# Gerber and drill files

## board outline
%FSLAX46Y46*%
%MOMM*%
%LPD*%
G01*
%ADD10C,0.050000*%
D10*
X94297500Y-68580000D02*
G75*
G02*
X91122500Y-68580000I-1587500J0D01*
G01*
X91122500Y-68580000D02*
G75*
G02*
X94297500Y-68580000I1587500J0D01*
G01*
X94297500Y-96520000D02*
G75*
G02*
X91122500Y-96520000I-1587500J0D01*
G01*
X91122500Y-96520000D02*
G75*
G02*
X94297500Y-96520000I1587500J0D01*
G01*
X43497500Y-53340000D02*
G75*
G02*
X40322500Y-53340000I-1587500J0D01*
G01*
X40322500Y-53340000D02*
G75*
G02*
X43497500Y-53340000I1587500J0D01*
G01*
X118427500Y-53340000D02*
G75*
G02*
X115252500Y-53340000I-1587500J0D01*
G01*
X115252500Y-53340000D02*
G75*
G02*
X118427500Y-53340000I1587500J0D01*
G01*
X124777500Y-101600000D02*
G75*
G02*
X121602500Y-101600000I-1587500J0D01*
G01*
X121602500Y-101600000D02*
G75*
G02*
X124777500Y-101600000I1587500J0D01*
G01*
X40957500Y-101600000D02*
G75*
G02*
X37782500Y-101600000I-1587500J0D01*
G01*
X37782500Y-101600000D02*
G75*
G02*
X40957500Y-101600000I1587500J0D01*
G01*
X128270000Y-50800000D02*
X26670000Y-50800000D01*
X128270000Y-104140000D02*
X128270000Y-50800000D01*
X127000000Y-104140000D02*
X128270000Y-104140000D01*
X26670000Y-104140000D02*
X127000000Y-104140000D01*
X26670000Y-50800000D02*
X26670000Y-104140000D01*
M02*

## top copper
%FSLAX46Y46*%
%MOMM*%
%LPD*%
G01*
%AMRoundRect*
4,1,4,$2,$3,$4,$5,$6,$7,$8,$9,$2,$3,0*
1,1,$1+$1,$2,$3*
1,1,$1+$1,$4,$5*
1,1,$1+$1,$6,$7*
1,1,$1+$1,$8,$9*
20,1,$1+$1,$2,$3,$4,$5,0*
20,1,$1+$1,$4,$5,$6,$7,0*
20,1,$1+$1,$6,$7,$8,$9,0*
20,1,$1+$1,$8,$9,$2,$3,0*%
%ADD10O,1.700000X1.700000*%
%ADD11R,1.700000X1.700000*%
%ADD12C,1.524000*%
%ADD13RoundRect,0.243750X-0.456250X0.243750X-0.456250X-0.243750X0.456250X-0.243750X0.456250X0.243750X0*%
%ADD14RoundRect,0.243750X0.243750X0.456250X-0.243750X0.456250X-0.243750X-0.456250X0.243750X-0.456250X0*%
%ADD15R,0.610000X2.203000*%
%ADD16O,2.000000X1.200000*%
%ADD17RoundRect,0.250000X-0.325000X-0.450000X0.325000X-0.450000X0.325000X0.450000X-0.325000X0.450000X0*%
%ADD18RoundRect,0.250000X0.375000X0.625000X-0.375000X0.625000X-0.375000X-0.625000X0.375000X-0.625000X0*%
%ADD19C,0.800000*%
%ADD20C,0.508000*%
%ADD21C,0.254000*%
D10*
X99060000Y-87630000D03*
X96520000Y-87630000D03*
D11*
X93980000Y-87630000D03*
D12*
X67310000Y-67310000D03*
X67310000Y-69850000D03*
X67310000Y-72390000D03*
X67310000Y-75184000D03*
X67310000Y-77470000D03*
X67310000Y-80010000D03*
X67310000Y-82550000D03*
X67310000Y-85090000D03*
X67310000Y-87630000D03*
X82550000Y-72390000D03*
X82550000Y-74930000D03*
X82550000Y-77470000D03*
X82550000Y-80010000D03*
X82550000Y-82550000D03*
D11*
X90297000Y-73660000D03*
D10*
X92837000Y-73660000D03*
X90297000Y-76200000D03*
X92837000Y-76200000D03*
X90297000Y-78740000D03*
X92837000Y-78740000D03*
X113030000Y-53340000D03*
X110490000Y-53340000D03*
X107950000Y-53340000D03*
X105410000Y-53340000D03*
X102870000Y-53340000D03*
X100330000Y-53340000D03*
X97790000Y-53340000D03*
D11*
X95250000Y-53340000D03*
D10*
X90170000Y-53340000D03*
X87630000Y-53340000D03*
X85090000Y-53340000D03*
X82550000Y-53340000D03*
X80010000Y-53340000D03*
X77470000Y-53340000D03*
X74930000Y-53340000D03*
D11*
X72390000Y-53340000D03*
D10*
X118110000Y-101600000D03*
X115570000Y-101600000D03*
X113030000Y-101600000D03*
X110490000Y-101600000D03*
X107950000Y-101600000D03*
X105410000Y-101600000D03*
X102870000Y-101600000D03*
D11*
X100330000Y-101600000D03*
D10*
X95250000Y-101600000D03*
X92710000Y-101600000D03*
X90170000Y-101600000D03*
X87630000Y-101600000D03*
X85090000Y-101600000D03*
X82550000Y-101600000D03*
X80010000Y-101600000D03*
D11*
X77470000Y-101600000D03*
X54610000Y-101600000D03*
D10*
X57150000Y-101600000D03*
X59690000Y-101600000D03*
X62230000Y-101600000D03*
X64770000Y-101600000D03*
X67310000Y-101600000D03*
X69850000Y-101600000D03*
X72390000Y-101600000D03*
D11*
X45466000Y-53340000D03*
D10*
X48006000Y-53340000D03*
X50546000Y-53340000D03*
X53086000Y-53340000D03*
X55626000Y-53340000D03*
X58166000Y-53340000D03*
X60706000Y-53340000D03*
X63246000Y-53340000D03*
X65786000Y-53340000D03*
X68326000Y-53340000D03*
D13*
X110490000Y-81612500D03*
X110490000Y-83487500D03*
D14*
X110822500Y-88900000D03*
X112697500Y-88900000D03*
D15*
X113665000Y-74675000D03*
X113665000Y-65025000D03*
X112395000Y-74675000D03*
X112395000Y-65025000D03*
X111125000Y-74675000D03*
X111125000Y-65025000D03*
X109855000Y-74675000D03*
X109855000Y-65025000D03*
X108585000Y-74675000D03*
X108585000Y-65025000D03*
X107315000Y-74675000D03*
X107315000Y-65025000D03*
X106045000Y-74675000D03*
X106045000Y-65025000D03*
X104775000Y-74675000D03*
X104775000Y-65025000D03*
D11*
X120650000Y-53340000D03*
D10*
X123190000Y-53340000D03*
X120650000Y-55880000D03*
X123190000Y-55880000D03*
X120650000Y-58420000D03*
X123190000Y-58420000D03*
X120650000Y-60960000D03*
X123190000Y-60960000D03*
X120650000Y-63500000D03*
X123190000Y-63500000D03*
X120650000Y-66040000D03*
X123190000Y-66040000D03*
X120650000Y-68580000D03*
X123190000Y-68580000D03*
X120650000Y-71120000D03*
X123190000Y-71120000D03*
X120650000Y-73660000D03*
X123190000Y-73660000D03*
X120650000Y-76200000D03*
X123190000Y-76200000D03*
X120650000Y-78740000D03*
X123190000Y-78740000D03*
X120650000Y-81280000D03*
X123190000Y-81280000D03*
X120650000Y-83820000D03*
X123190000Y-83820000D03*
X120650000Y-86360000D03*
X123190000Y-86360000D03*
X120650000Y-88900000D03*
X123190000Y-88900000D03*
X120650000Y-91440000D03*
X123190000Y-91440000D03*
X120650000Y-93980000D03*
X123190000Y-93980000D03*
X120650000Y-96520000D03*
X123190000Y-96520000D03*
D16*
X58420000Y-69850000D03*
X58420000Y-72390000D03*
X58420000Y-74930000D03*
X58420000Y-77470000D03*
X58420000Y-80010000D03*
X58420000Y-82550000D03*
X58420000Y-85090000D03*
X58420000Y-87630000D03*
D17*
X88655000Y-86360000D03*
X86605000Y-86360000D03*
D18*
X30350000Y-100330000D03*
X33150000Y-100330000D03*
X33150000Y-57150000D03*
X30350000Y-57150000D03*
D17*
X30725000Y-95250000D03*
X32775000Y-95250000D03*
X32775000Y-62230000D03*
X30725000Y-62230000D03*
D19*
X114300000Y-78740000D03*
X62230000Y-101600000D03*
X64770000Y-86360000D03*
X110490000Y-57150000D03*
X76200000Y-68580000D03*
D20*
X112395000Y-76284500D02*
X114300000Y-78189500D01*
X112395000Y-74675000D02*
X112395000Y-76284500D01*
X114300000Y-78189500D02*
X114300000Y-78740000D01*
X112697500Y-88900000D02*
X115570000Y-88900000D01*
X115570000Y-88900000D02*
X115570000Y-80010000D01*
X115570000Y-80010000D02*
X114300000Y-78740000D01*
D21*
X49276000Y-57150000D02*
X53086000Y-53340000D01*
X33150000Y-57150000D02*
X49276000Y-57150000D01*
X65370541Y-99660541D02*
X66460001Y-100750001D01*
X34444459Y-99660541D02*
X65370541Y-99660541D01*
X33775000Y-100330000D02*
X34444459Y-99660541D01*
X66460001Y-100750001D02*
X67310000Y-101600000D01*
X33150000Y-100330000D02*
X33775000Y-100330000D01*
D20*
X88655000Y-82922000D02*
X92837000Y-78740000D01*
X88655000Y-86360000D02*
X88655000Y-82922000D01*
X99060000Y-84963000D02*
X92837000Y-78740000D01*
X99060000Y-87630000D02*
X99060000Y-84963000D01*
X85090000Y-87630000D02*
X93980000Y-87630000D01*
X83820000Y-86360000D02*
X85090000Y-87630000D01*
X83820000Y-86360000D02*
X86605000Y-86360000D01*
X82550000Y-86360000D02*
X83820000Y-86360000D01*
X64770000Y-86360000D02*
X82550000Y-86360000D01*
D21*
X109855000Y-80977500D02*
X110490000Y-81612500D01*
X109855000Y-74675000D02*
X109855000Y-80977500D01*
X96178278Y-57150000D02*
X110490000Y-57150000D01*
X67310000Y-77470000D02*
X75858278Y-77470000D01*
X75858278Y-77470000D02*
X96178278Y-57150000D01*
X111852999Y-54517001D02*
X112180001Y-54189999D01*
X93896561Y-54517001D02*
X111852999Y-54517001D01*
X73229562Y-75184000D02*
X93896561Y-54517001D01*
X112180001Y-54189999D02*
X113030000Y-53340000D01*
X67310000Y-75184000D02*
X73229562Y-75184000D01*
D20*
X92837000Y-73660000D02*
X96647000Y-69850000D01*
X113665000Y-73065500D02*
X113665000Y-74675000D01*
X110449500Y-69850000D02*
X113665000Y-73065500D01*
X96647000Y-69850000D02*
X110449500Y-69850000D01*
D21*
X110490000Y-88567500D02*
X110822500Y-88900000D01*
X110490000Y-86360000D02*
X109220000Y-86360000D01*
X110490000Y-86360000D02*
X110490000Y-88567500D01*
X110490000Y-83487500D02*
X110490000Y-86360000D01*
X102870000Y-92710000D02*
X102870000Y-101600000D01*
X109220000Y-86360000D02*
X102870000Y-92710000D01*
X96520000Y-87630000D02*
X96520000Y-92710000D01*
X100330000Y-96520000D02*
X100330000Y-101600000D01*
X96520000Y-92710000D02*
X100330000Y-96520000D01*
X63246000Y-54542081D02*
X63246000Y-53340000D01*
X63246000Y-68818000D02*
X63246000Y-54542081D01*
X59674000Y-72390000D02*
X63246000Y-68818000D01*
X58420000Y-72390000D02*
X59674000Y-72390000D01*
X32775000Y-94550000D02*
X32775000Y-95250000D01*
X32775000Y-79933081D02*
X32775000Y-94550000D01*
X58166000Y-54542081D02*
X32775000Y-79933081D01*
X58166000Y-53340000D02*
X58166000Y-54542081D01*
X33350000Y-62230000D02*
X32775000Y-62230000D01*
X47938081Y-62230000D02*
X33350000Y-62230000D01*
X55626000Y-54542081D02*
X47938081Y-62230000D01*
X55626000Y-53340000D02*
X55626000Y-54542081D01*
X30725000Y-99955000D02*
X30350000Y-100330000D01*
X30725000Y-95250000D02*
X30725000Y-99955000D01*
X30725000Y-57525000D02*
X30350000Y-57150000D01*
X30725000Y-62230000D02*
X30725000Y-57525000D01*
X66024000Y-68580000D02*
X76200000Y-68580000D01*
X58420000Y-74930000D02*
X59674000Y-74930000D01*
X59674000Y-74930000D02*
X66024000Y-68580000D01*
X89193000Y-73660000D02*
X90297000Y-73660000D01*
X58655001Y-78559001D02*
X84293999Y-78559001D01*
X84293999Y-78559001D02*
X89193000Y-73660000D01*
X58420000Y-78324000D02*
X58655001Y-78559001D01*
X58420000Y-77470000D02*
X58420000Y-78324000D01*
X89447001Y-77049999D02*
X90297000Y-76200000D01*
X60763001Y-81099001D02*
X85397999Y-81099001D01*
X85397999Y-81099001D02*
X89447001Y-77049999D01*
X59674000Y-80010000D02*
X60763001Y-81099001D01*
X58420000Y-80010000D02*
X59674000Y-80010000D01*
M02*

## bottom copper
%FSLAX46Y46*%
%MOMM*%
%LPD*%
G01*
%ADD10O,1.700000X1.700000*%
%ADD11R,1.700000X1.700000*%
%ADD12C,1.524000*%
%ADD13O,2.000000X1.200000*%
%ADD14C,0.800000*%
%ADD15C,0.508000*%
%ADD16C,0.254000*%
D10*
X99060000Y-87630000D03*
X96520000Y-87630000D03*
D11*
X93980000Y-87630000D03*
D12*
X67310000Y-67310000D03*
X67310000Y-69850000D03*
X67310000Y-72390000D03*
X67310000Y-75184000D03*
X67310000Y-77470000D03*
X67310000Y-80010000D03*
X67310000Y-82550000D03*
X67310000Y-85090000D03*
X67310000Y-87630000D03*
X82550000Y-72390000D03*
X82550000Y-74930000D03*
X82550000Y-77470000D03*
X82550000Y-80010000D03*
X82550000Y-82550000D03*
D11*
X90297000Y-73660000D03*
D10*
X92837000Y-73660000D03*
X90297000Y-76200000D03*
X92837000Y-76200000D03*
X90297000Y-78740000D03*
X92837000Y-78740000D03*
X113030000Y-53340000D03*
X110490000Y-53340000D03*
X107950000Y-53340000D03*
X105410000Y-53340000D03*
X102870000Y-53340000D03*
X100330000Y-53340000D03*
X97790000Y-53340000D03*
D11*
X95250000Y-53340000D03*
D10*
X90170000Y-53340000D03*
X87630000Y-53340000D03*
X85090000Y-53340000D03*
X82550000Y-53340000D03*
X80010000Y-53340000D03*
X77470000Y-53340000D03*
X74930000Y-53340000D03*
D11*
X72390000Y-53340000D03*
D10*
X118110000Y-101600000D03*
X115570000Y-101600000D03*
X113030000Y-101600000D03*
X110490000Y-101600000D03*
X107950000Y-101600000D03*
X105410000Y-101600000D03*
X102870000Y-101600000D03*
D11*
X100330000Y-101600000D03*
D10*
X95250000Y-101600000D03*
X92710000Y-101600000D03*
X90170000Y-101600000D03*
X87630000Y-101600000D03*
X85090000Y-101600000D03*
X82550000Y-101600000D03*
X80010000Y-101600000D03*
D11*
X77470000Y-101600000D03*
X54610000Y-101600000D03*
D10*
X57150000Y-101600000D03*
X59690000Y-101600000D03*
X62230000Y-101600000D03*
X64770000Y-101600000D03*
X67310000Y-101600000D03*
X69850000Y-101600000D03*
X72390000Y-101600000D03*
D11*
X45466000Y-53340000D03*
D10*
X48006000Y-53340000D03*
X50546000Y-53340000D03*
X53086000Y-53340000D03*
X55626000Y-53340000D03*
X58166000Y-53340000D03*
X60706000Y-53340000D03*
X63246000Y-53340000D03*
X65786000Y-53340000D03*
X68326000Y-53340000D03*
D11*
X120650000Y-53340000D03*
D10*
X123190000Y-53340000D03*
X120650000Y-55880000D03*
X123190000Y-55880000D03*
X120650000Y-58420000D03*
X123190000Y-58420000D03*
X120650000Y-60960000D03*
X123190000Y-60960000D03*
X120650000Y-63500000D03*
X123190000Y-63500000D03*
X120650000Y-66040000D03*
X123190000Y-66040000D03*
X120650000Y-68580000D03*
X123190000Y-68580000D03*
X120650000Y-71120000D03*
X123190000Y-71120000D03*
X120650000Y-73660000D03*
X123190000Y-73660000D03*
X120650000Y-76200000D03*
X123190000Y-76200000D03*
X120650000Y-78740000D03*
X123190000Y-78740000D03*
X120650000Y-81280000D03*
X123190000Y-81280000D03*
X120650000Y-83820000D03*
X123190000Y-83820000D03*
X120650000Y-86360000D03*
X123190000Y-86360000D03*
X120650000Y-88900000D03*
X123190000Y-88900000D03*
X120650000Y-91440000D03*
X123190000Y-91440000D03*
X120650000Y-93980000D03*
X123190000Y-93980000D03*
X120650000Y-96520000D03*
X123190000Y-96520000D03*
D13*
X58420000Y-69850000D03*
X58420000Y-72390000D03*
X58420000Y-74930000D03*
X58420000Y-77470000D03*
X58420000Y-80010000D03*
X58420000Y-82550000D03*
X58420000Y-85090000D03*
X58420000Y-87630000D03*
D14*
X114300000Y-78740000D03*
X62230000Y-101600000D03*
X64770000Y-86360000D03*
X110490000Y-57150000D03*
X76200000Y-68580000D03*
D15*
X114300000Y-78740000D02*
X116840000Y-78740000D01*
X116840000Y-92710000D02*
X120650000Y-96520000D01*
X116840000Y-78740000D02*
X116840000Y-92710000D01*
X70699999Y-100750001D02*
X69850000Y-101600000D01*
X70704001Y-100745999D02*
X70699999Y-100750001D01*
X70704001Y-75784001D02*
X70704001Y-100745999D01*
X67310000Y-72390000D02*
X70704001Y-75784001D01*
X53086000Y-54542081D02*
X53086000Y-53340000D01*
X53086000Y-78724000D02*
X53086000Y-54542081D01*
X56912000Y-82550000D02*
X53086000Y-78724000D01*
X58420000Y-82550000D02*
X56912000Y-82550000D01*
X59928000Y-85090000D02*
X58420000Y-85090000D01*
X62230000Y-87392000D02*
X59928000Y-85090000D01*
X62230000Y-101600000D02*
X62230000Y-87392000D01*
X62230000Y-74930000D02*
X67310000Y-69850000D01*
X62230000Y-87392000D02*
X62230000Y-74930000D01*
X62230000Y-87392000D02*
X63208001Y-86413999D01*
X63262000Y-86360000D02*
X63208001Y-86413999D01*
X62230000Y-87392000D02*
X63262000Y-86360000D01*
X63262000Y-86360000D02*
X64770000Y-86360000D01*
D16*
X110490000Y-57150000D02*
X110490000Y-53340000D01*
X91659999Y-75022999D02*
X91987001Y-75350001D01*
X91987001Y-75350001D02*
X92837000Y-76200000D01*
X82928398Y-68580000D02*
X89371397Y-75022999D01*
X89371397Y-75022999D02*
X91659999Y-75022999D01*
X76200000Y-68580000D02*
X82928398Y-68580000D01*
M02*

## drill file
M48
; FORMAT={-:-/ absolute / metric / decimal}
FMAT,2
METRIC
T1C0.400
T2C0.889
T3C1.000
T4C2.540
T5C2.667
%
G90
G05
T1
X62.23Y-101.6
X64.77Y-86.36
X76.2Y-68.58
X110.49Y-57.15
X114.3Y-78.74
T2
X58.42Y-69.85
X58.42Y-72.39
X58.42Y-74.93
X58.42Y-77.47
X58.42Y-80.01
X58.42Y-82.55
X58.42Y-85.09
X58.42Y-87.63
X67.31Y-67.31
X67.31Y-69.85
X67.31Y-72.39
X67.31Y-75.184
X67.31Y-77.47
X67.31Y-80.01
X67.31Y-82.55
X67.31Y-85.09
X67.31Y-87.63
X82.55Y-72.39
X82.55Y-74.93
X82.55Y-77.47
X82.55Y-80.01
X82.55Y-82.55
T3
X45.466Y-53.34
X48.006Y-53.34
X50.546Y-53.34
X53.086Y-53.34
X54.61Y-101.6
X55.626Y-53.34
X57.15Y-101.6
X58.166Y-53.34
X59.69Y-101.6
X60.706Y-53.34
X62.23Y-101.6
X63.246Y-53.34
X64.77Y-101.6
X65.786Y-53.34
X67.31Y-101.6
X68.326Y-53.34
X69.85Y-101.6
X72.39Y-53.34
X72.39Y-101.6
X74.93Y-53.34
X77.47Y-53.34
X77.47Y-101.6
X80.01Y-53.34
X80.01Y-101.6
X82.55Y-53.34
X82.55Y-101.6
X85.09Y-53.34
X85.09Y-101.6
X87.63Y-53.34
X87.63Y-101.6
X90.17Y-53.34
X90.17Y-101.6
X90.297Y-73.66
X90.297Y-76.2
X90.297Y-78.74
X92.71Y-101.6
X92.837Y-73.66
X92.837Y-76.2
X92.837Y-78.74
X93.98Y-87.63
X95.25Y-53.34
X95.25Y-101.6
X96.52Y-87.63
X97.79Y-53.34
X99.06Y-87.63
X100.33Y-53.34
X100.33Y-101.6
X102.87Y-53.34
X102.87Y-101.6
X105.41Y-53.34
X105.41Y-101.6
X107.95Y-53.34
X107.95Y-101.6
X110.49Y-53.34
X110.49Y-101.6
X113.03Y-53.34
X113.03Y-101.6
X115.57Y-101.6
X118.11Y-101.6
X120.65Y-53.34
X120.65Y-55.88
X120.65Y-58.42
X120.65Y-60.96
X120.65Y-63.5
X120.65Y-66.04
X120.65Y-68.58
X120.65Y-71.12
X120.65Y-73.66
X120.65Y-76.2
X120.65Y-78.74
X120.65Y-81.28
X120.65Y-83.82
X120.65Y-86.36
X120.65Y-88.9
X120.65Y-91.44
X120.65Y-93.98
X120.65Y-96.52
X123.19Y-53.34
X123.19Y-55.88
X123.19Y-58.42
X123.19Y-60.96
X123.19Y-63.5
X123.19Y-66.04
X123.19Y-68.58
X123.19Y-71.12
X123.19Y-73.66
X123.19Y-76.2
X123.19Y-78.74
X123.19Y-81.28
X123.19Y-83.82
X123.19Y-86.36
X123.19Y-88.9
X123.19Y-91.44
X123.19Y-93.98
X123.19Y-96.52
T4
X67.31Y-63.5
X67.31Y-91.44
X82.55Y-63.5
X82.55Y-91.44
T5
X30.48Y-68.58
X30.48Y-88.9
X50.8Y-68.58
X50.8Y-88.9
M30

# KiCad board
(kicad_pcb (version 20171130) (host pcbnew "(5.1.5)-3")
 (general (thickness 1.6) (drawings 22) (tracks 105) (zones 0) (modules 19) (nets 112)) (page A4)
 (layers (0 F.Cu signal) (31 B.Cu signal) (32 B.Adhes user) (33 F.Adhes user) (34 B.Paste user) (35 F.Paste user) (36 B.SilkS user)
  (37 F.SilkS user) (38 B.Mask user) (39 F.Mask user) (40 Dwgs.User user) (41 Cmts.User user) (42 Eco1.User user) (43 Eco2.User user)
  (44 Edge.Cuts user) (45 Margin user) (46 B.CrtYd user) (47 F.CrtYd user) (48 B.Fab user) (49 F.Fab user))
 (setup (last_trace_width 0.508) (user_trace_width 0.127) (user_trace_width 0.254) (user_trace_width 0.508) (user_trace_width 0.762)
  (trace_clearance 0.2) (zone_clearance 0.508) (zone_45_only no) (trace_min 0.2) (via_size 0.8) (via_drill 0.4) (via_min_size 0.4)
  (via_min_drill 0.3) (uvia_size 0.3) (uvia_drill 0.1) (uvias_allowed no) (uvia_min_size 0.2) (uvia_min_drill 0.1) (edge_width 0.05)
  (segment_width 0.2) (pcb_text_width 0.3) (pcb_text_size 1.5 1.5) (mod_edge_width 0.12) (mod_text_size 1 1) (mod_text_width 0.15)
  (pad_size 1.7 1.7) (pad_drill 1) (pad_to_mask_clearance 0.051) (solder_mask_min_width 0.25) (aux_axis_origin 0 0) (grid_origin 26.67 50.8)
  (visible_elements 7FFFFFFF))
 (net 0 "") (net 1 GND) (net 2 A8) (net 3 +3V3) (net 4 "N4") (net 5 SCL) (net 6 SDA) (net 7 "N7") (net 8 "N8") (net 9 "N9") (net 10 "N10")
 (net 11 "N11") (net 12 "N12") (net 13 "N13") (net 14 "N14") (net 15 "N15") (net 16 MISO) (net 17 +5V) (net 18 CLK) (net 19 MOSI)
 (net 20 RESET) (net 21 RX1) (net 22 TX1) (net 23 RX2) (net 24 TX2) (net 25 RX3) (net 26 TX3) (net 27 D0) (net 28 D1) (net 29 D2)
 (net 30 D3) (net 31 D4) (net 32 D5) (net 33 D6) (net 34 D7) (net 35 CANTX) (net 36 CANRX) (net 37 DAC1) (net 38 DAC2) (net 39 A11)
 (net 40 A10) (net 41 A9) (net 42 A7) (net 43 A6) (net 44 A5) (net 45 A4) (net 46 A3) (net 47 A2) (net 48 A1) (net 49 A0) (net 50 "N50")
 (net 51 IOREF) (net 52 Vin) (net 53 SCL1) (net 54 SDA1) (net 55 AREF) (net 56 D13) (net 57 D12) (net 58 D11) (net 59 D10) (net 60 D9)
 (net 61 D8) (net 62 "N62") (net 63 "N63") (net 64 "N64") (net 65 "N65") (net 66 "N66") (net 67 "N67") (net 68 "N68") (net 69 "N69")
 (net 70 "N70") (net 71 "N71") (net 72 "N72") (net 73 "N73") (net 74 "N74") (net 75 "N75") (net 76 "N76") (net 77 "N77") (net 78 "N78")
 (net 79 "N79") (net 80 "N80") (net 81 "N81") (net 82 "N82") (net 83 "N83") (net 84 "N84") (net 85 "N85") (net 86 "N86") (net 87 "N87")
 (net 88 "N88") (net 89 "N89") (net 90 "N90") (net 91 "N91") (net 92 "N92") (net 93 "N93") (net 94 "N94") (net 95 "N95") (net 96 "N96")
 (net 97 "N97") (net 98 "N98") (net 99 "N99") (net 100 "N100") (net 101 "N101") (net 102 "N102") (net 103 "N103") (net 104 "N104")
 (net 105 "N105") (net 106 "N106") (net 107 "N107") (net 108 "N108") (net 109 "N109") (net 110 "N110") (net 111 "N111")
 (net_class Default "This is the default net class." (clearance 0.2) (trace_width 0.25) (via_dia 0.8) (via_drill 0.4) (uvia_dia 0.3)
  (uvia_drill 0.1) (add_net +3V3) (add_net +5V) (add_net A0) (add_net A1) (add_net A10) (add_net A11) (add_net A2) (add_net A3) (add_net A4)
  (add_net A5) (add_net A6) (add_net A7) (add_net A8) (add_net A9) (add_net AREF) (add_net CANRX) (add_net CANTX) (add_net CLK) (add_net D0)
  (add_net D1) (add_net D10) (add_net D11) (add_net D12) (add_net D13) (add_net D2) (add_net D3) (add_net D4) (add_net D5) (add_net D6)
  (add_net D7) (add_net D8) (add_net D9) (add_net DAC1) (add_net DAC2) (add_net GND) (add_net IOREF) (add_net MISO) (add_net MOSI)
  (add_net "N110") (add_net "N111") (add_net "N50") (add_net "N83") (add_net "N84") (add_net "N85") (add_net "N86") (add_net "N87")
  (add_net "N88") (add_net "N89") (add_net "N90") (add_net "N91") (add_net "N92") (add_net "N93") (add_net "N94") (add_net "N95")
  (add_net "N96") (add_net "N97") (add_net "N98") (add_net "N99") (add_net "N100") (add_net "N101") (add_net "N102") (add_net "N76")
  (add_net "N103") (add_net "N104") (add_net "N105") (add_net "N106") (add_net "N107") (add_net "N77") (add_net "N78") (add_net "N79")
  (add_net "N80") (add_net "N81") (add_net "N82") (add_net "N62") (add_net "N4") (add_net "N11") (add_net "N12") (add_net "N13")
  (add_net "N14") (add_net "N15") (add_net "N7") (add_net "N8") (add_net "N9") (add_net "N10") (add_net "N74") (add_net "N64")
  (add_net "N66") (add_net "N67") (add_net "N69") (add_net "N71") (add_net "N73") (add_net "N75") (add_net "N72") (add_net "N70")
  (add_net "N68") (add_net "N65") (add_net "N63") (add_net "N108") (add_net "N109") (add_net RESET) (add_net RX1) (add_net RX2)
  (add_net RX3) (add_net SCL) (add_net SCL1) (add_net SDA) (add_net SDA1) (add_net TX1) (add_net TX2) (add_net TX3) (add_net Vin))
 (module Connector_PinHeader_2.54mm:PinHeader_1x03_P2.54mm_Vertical (layer F.Cu) (at 93.98 87.63 90)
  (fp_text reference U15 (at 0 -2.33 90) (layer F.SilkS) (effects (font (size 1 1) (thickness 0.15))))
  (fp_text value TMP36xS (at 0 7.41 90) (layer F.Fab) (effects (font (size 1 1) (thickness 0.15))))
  (pad 3 thru_hole oval (at 0 5.08 90) (size 1.7 1.7) (drill 1) (layers *.Cu *.Mask) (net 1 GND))
  (pad 2 thru_hole oval (at 0 2.54 90) (size 1.7 1.7) (drill 1) (layers *.Cu *.Mask) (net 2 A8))
  (pad 1 thru_hole rect (at 0 0 90) (size 1.7 1.7) (drill 1) (layers *.Cu *.Mask) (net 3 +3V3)))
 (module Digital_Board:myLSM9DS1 (layer F.Cu) (at 74.93 77.47)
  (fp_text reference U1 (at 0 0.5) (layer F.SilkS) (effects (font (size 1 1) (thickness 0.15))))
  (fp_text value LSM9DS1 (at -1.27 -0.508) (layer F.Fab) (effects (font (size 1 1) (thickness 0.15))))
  (pad 1 thru_hole circle (at -7.62 -10.16) (size 1.524 1.524) (drill 0.889) (layers *.Cu *.Mask) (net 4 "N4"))
  (pad 2 thru_hole circle (at -7.62 -7.62) (size 1.524 1.524) (drill 0.889) (layers *.Cu *.Mask) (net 3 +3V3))
  (pad 3 thru_hole circle (at -7.62 -5.08) (size 1.524 1.524) (drill 0.889) (layers *.Cu *.Mask) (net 1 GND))
  (pad 4 thru_hole circle (at -7.62 -2.286) (size 1.524 1.524) (drill 0.889) (layers *.Cu *.Mask) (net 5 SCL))
  (pad 5 thru_hole circle (at -7.62 0) (size 1.524 1.524) (drill 0.889) (layers *.Cu *.Mask) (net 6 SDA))
  (pad 6 thru_hole circle (at -7.62 2.54) (size 1.524 1.524) (drill 0.889) (layers *.Cu *.Mask) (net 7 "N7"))
  (pad 7 thru_hole circle (at -7.62 5.08) (size 1.524 1.524) (drill 0.889) (layers *.Cu *.Mask) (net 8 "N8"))
  (pad 8 thru_hole circle (at -7.62 7.62) (size 1.524 1.524) (drill 0.889) (layers *.Cu *.Mask) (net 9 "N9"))
  (pad 9 thru_hole circle (at -7.62 10.16) (size 1.524 1.524) (drill 0.889) (layers *.Cu *.Mask Eco2.User) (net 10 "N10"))
  (pad 10 thru_hole circle (at 7.62 -5.08) (size 1.524 1.524) (drill 0.889) (layers *.Cu *.Mask) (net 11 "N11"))
  (pad 11 thru_hole circle (at 7.62 -2.54) (size 1.524 1.524) (drill 0.889) (layers *.Cu *.Mask) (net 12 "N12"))
  (pad 12 thru_hole circle (at 7.62 0) (size 1.524 1.524) (drill 0.889) (layers *.Cu *.Mask) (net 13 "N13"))
  (pad 13 thru_hole circle (at 7.62 2.54) (size 1.524 1.524) (drill 0.889) (layers *.Cu *.Mask) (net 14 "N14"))
  (pad 14 thru_hole circle (at 7.62 5.08) (size 1.524 1.524) (drill 0.889) (layers *.Cu *.Mask) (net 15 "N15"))
  (pad "" np_thru_hole circle (at -7.62 -13.97) (size 2.54 2.54) (drill 2.54) (layers *.Cu *.Mask))
  (pad "" np_thru_hole circle (at 7.62 -13.97) (size 2.54 2.54) (drill 2.54) (layers *.Cu *.Mask))
  (pad "" np_thru_hole circle (at -7.62 13.97) (size 2.54 2.54) (drill 2.54) (layers *.Cu *.Mask))
  (pad "" np_thru_hole circle (at 7.62 13.97) (size 2.54 2.54) (drill 2.54) (layers *.Cu *.Mask)))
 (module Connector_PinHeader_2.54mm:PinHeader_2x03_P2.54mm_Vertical (layer F.Cu) (at 90.297 73.66)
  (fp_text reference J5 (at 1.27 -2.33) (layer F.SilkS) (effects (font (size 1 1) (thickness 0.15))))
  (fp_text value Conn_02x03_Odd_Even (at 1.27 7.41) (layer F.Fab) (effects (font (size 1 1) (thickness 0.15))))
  (pad 1 thru_hole rect (at 0 0) (size 1.7 1.7) (drill 1) (layers *.Cu *.Mask) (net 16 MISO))
  (pad 2 thru_hole oval (at 2.54 0) (size 1.7 1.7) (drill 1) (layers *.Cu *.Mask) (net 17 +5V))
  (pad 3 thru_hole oval (at 0 2.54) (size 1.7 1.7) (drill 1) (layers *.Cu *.Mask) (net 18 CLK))
  (pad 4 thru_hole oval (at 2.54 2.54) (size 1.7 1.7) (drill 1) (layers *.Cu *.Mask) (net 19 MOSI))
  (pad 5 thru_hole oval (at 0 5.08) (size 1.7 1.7) (drill 1) (layers *.Cu *.Mask) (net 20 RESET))
  (pad 6 thru_hole oval (at 2.54 5.08) (size 1.7 1.7) (drill 1) (layers *.Cu *.Mask) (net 1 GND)))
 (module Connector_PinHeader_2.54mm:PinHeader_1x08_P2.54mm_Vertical (layer F.Cu) (at 95.25 53.34 90)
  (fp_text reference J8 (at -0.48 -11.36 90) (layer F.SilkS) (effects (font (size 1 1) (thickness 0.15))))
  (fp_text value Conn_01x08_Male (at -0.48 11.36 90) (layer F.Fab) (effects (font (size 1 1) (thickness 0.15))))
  (pad 8 thru_hole oval (at 0 17.78 90) (size 1.7 1.7) (drill 1) (layers *.Cu *.Mask) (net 5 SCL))
  (pad 7 thru_hole oval (at 0 15.24 90) (size 1.7 1.7) (drill 1) (layers *.Cu *.Mask) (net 6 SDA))
  (pad 6 thru_hole oval (at 0 12.7 90) (size 1.7 1.7) (drill 1) (layers *.Cu *.Mask) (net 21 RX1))
  (pad 5 thru_hole oval (at 0 10.16 90) (size 1.7 1.7) (drill 1) (layers *.Cu *.Mask) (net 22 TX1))
  (pad 4 thru_hole oval (at 0 7.62 90) (size 1.7 1.7) (drill 1) (layers *.Cu *.Mask) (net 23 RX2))
  (pad 3 thru_hole oval (at 0 5.08 90) (size 1.7 1.7) (drill 1) (layers *.Cu *.Mask) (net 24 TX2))
  (pad 2 thru_hole oval (at 0 2.54 90) (size 1.7 1.7) (drill 1) (layers *.Cu *.Mask) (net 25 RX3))
  (pad 1 thru_hole rect (at 0 0 90) (size 1.7 1.7) (drill 1) (layers *.Cu *.Mask) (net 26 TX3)))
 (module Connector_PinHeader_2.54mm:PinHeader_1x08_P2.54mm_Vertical (layer F.Cu) (at 72.39 53.34 90)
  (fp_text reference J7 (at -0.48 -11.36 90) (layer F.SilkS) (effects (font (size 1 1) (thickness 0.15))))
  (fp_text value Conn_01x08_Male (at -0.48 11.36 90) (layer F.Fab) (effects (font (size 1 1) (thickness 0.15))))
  (pad 8 thru_hole oval (at 0 17.78 90) (size 1.7 1.7) (drill 1) (layers *.Cu *.Mask) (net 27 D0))
  (pad 7 thru_hole oval (at 0 15.24 90) (size 1.7 1.7) (drill 1) (layers *.Cu *.Mask) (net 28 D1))
  (pad 6 thru_hole oval (at 0 12.7 90) (size 1.7 1.7) (drill 1) (layers *.Cu *.Mask) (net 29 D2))
  (pad 5 thru_hole oval (at 0 10.16 90) (size 1.7 1.7) (drill 1) (layers *.Cu *.Mask) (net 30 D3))
  (pad 4 thru_hole oval (at 0 7.62 90) (size 1.7 1.7) (drill 1) (layers *.Cu *.Mask) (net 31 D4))
  (pad 3 thru_hole oval (at 0 5.08 90) (size 1.7 1.7) (drill 1) (layers *.Cu *.Mask) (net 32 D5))
  (pad 2 thru_hole oval (at 0 2.54 90) (size 1.7 1.7) (drill 1) (layers *.Cu *.Mask) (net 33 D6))
  (pad 1 thru_hole rect (at 0 0 90) (size 1.7 1.7) (drill 1) (layers *.Cu *.Mask) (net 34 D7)))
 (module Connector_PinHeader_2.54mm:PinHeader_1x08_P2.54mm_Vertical (layer F.Cu) (at 100.33 101.6 90)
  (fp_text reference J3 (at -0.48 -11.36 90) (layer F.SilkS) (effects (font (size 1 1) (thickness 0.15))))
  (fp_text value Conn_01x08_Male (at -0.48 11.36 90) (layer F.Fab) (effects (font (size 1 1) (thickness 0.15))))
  (pad 8 thru_hole oval (at 0 17.78 90) (size 1.7 1.7) (drill 1) (layers *.Cu *.Mask) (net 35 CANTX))
  (pad 7 thru_hole oval (at 0 15.24 90) (size 1.7 1.7) (drill 1) (layers *.Cu *.Mask) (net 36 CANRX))
  (pad 6 thru_hole oval (at 0 12.7 90) (size 1.7 1.7) (drill 1) (layers *.Cu *.Mask) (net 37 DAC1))
  (pad 5 thru_hole oval (at 0 10.16 90) (size 1.7 1.7) (drill 1) (layers *.Cu *.Mask) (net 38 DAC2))
  (pad 4 thru_hole oval (at 0 7.62 90) (size 1.7 1.7) (drill 1) (layers *.Cu *.Mask) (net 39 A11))
  (pad 3 thru_hole oval (at 0 5.08 90) (size 1.7 1.7) (drill 1) (layers *.Cu *.Mask) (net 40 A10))
  (pad 2 thru_hole oval (at 0 2.54 90) (size 1.7 1.7) (drill 1) (layers *.Cu *.Mask) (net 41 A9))
  (pad 1 thru_hole rect (at 0 0 90) (size 1.7 1.7) (drill 1) (layers *.Cu *.Mask) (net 2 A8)))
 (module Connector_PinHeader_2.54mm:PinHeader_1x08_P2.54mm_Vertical (layer F.Cu) (at 77.47 101.6 90)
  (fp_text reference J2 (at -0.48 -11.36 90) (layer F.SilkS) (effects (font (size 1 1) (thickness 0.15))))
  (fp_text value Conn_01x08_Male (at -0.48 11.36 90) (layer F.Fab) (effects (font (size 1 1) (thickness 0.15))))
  (pad 8 thru_hole oval (at 0 17.78 90) (size 1.7 1.7) (drill 1) (layers *.Cu *.Mask) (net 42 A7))
  (pad 7 thru_hole oval (at 0 15.24 90) (size 1.7 1.7) (drill 1) (layers *.Cu *.Mask) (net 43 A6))
  (pad 6 thru_hole oval (at 0 12.7 90) (size 1.7 1.7) (drill 1) (layers *.Cu *.Mask) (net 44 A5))
  (pad 5 thru_hole oval (at 0 10.16 90) (size 1.7 1.7) (drill 1) (layers *.Cu *.Mask) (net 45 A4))
  (pad 4 thru_hole oval (at 0 7.62 90) (size 1.7 1.7) (drill 1) (layers *.Cu *.Mask) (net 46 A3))
  (pad 3 thru_hole oval (at 0 5.08 90) (size 1.7 1.7) (drill 1) (layers *.Cu *.Mask) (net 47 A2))
  (pad 2 thru_hole oval (at 0 2.54 90) (size 1.7 1.7) (drill 1) (layers *.Cu *.Mask) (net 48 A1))
  (pad 1 thru_hole rect (at 0 0 90) (size 1.7 1.7) (drill 1) (layers *.Cu *.Mask) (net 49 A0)))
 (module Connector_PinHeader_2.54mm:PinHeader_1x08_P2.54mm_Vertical (layer F.Cu) (at 54.61 101.6 90)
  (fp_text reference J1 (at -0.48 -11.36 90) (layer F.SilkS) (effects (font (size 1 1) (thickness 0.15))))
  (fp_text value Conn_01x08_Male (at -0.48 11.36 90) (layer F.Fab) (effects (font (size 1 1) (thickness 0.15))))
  (pad 1 thru_hole rect (at 0 0 90) (size 1.7 1.7) (drill 1) (layers *.Cu *.Mask) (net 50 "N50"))
  (pad 2 thru_hole oval (at 0 2.54 90) (size 1.7 1.7) (drill 1) (layers *.Cu *.Mask) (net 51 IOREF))
  (pad 3 thru_hole oval (at 0 5.08 90) (size 1.7 1.7) (drill 1) (layers *.Cu *.Mask) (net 20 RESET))
  (pad 4 thru_hole oval (at 0 7.62 90) (size 1.7 1.7) (drill 1) (layers *.Cu *.Mask) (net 3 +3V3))
  (pad 5 thru_hole oval (at 0 10.16 90) (size 1.7 1.7) (drill 1) (layers *.Cu *.Mask) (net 17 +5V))
  (pad 6 thru_hole oval (at 0 12.7 90) (size 1.7 1.7) (drill 1) (layers *.Cu *.Mask) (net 1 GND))
  (pad 7 thru_hole oval (at 0 15.24 90) (size 1.7 1.7) (drill 1) (layers *.Cu *.Mask) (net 1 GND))
  (pad 8 thru_hole oval (at 0 17.78 90) (size 1.7 1.7) (drill 1) (layers *.Cu *.Mask) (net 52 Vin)))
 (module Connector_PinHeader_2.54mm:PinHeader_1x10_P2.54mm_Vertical (layer F.Cu) (at 45.466 53.34 90)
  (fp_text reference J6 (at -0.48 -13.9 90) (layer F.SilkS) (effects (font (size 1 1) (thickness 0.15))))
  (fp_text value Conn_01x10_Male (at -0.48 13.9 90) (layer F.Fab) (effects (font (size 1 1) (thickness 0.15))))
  (pad 1 thru_hole rect (at 0 0 90) (size 1.7 1.7) (drill 1) (layers *.Cu *.Mask) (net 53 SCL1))
  (pad 2 thru_hole oval (at 0 2.54 90) (size 1.7 1.7) (drill 1) (layers *.Cu *.Mask) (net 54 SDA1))
  (pad 3 thru_hole oval (at 0 5.08 90) (size 1.7 1.7) (drill 1) (layers *.Cu *.Mask) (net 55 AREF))
  (pad 4 thru_hole oval (at 0 7.62 90) (size 1.7 1.7) (drill 1) (layers *.Cu *.Mask) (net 1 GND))
  (pad 5 thru_hole oval (at 0 10.16 90) (size 1.7 1.7) (drill 1) (layers *.Cu *.Mask) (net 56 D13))
  (pad 6 thru_hole oval (at 0 12.7 90) (size 1.7 1.7) (drill 1) (layers *.Cu *.Mask) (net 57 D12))
  (pad 7 thru_hole oval (at 0 15.24 90) (size 1.7 1.7) (drill 1) (layers *.Cu *.Mask) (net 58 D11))
  (pad 8 thru_hole oval (at 0 17.78 90) (size 1.7 1.7) (drill 1) (layers *.Cu *.Mask) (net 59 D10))
  (pad 9 thru_hole oval (at 0 20.32 90) (size 1.7 1.7) (drill 1) (layers *.Cu *.Mask) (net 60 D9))
  (pad 10 thru_hole oval (at 0 22.86 90) (size 1.7 1.7) (drill 1) (layers *.Cu *.Mask) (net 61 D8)))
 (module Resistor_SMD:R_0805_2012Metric (layer F.Cu) (at 110.49 82.55 270)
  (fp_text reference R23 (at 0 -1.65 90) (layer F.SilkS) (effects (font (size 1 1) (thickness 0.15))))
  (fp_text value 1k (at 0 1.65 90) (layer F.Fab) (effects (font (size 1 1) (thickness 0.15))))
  (pad 1 smd roundrect (at -0.9375 0 270) (size 0.975 1.4) (layers F.Cu F.Paste F.Mask) (roundrect_rratio 0.25) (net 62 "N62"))
  (pad 2 smd roundrect (at 0.9375 0 270) (size 0.975 1.4) (layers F.Cu F.Paste F.Mask) (roundrect_rratio 0.25) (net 41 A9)))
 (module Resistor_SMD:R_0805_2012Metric (layer F.Cu) (at 111.76 88.9 180)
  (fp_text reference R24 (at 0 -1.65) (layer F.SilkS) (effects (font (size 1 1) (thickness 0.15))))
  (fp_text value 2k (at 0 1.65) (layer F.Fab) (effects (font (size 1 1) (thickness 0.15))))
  (pad 2 smd roundrect (at 0.9375 0 180) (size 0.975 1.4) (layers F.Cu F.Paste F.Mask) (roundrect_rratio 0.25) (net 41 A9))
  (pad 1 smd roundrect (at -0.9375 0 180) (size 0.975 1.4) (layers F.Cu F.Paste F.Mask) (roundrect_rratio 0.25) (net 1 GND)))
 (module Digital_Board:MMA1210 (layer F.Cu) (at 109.22 69.85)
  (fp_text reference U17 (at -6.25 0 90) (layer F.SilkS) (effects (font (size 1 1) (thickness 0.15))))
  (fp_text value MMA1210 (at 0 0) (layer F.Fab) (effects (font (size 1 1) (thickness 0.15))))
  (pad 8 smd rect (at 4.445 4.825) (size 0.61 2.203) (layers F.Cu F.Paste F.Mask) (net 17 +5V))
  (pad 9 smd rect (at 4.445 -4.825) (size 0.61 2.203) (layers F.Cu F.Paste F.Mask) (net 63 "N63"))
  (pad 7 smd rect (at 3.175 4.825) (size 0.61 2.203) (layers F.Cu F.Paste F.Mask) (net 1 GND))
  (pad 10 smd rect (at 3.175 -4.825) (size 0.61 2.203) (layers F.Cu F.Paste F.Mask) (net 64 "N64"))
  (pad 6 smd rect (at 1.905 4.825) (size 0.61 2.203) (layers F.Cu F.Paste F.Mask) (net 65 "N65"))
  (pad 11 smd rect (at 1.905 -4.825) (size 0.61 2.203) (layers F.Cu F.Paste F.Mask) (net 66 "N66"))
  (pad 5 smd rect (at 0.635 4.825) (size 0.61 2.203) (layers F.Cu F.Paste F.Mask) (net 62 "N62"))
  (pad 12 smd rect (at 0.635 -4.825) (size 0.61 2.203) (layers F.Cu F.Paste F.Mask) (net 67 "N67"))
  (pad 4 smd rect (at -0.635 4.825) (size 0.61 2.203) (layers F.Cu F.Paste F.Mask) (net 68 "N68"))
  (pad 13 smd rect (at -0.635 -4.825) (size 0.61 2.203) (layers F.Cu F.Paste F.Mask) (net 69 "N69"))
  (pad 3 smd rect (at -1.905 4.825) (size 0.61 2.203) (layers F.Cu F.Paste F.Mask) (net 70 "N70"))
  (pad 14 smd rect (at -1.905 -4.825) (size 0.61 2.203) (layers F.Cu F.Paste F.Mask) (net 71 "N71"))
  (pad 2 smd rect (at -3.175 4.825) (size 0.61 2.203) (layers F.Cu F.Paste F.Mask) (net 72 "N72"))
  (pad 15 smd rect (at -3.175 -4.825) (size 0.61 2.203) (layers F.Cu F.Paste F.Mask) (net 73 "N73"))
  (pad 1 smd rect (at -4.445 4.825) (size 0.61 2.203) (layers F.Cu F.Paste F.Mask) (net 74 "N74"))
  (pad 16 smd rect (at -4.445 -4.825) (size 0.61 2.203) (layers F.Cu F.Paste F.Mask) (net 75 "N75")))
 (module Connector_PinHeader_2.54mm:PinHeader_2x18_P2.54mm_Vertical (layer F.Cu) (at 120.65 53.34)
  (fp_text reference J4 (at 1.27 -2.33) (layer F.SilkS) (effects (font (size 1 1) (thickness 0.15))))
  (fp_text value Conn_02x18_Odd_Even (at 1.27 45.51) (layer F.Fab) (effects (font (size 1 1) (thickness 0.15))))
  (pad 1 thru_hole rect (at 0 0) (size 1.7 1.7) (drill 1) (layers *.Cu *.Mask) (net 17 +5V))
  (pad 2 thru_hole oval (at 2.54 0) (size 1.7 1.7) (drill 1) (layers *.Cu *.Mask) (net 17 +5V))
  (pad 3 thru_hole oval (at 0 2.54) (size 1.7 1.7) (drill 1) (layers *.Cu *.Mask) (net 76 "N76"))
  (pad 4 thru_hole oval (at 2.54 2.54) (size 1.7 1.7) (drill 1) (layers *.Cu *.Mask) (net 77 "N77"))
  (pad 5 thru_hole oval (at 0 5.08) (size 1.7 1.7) (drill 1) (layers *.Cu *.Mask) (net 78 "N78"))
  (pad 6 thru_hole oval (at 2.54 5.08) (size 1.7 1.7) (drill 1) (layers *.Cu *.Mask) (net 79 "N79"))
  (pad 7 thru_hole oval (at 0 7.62) (size 1.7 1.7) (drill 1) (layers *.Cu *.Mask) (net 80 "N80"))
  (pad 8 thru_hole oval (at 2.54 7.62) (size 1.7 1.7) (drill 1) (layers *.Cu *.Mask) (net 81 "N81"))
  (pad 9 thru_hole oval (at 0 10.16) (size 1.7 1.7) (drill 1) (layers *.Cu *.Mask) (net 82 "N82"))
  (pad 10 thru_hole oval (at 2.54 10.16) (size 1.7 1.7) (drill 1) (layers *.Cu *.Mask) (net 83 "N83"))
  (pad 11 thru_hole oval (at 0 12.7) (size 1.7 1.7) (drill 1) (layers *.Cu *.Mask) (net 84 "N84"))
  (pad 12 thru_hole oval (at 2.54 12.7) (size 1.7 1.7) (drill 1) (layers *.Cu *.Mask) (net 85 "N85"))
  (pad 13 thru_hole oval (at 0 15.24) (size 1.7 1.7) (drill 1) (layers *.Cu *.Mask) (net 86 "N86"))
  (pad 14 thru_hole oval (at 2.54 15.24) (size 1.7 1.7) (drill 1) (layers *.Cu *.Mask) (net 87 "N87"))
  (pad 15 thru_hole oval (at 0 17.78) (size 1.7 1.7) (drill 1) (layers *.Cu *.Mask) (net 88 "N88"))
  (pad 16 thru_hole oval (at 2.54 17.78) (size 1.7 1.7) (drill 1) (layers *.Cu *.Mask) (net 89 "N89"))
  (pad 17 thru_hole oval (at 0 20.32) (size 1.7 1.7) (drill 1) (layers *.Cu *.Mask) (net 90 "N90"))
  (pad 18 thru_hole oval (at 2.54 20.32) (size 1.7 1.7) (drill 1) (layers *.Cu *.Mask) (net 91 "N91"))
  (pad 19 thru_hole oval (at 0 22.86) (size 1.7 1.7) (drill 1) (layers *.Cu *.Mask) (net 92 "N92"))
  (pad 20 thru_hole oval (at 2.54 22.86) (size 1.7 1.7) (drill 1) (layers *.Cu *.Mask) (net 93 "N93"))
  (pad 21 thru_hole oval (at 0 25.4) (size 1.7 1.7) (drill 1) (layers *.Cu *.Mask) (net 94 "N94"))
  (pad 22 thru_hole oval (at 2.54 25.4) (size 1.7 1.7) (drill 1) (layers *.Cu *.Mask) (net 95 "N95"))
  (pad 23 thru_hole oval (at 0 27.94) (size 1.7 1.7) (drill 1) (layers *.Cu *.Mask) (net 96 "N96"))
  (pad 24 thru_hole oval (at 2.54 27.94) (size 1.7 1.7) (drill 1) (layers *.Cu *.Mask) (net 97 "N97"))
  (pad 25 thru_hole oval (at 0 30.48) (size 1.7 1.7) (drill 1) (layers *.Cu *.Mask) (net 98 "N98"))
  (pad 26 thru_hole oval (at 2.54 30.48) (size 1.7 1.7) (drill 1) (layers *.Cu *.Mask) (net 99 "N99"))
  (pad 27 thru_hole oval (at 0 33.02) (size 1.7 1.7) (drill 1) (layers *.Cu *.Mask) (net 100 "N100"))
  (pad 28 thru_hole oval (at 2.54 33.02) (size 1.7 1.7) (drill 1) (layers *.Cu *.Mask) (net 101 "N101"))
  (pad 29 thru_hole oval (at 0 35.56) (size 1.7 1.7) (drill 1) (layers *.Cu *.Mask) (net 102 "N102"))
  (pad 30 thru_hole oval (at 2.54 35.56) (size 1.7 1.7) (drill 1) (layers *.Cu *.Mask) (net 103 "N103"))
  (pad 31 thru_hole oval (at 0 38.1) (size 1.7 1.7) (drill 1) (layers *.Cu *.Mask) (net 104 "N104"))
  (pad 32 thru_hole oval (at 2.54 38.1) (size 1.7 1.7) (drill 1) (layers *.Cu *.Mask) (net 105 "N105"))
  (pad 33 thru_hole oval (at 0 40.64) (size 1.7 1.7) (drill 1) (layers *.Cu *.Mask) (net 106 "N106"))
  (pad 34 thru_hole oval (at 2.54 40.64) (size 1.7 1.7) (drill 1) (layers *.Cu *.Mask) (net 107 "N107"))
  (pad 35 thru_hole oval (at 0 43.18) (size 1.7 1.7) (drill 1) (layers *.Cu *.Mask) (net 1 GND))
  (pad 36 thru_hole oval (at 2.54 43.18) (size 1.7 1.7) (drill 1) (layers *.Cu *.Mask) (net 1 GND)))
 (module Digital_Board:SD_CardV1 (layer F.Cu) (at 59.69 66.04 270)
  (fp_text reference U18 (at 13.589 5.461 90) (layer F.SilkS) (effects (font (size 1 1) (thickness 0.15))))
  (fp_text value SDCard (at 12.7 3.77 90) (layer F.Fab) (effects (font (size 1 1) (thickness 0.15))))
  (pad 1 thru_hole oval (at 3.81 1.27 270) (size 1.2 2) (drill 0.889) (layers *.Cu *.Mask) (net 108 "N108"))
  (pad 2 thru_hole oval (at 6.35 1.27 270) (size 1.2 2) (drill 0.889) (layers *.Cu *.Mask) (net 59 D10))
  (pad 3 thru_hole oval (at 8.89 1.27 270) (size 1.2 2) (drill 0.889) (layers *.Cu *.Mask) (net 19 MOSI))
  (pad 4 thru_hole oval (at 11.43 1.27 270) (size 1.2 2) (drill 0.889) (layers *.Cu *.Mask) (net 16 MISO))
  (pad 5 thru_hole oval (at 13.97 1.27 270) (size 1.2 2) (drill 0.889) (layers *.Cu *.Mask) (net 18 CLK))
  (pad 6 thru_hole oval (at 16.51 1.27 270) (size 1.2 2) (drill 0.889) (layers *.Cu *.Mask) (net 1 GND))
  (pad 7 thru_hole oval (at 19.05 1.27 270) (size 1.2 2) (drill 0.889) (layers *.Cu *.Mask) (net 3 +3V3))
  (pad 8 thru_hole oval (at 21.59 1.27 270) (size 1.2 2) (drill 0.889) (layers *.Cu *.Mask) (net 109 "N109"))
  (pad "" np_thru_hole circle (at 2.54 8.89 270) (size 2.667 2.667) (drill 2.667) (layers *.Cu *.Mask))
  (pad "" np_thru_hole circle (at 22.86 8.89 270) (size 2.667 2.667) (drill 2.667) (layers *.Cu *.Mask))
  (pad "" np_thru_hole circle (at 22.86 29.21 270) (size 2.667 2.667) (drill 2.667) (layers *.Cu *.Mask))
  (pad "" np_thru_hole circle (at 2.54 29.21 270) (size 2.667 2.667) (drill 2.667) (layers *.Cu *.Mask)))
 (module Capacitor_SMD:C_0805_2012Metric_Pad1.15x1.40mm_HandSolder (layer F.Cu) (at 87.63 86.36)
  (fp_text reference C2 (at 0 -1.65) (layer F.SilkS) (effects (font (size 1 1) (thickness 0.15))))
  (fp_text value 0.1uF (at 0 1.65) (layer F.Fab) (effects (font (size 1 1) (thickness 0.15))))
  (pad 2 smd roundrect (at 1.025 0) (size 1.15 1.4) (layers F.Cu F.Paste F.Mask) (roundrect_rratio 0.217391) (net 1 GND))
  (pad 1 smd roundrect (at -1.025 0) (size 1.15 1.4) (layers F.Cu F.Paste F.Mask) (roundrect_rratio 0.217391) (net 3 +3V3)))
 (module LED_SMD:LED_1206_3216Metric (layer F.Cu) (at 31.75 100.33 180)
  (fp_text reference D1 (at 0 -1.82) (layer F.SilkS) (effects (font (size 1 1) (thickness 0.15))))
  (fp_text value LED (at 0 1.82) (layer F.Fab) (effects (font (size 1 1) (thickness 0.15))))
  (pad 2 smd roundrect (at 1.4 0 180) (size 1.25 1.75) (layers F.Cu F.Paste F.Mask) (roundrect_rratio 0.2) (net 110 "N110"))
  (pad 1 smd roundrect (at -1.4 0 180) (size 1.25 1.75) (layers F.Cu F.Paste F.Mask) (roundrect_rratio 0.2) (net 1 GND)))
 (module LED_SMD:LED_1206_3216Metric (layer F.Cu) (at 31.75 57.15 180)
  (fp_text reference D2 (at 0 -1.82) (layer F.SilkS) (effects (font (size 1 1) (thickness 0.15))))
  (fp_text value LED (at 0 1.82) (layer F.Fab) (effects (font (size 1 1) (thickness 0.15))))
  (pad 1 smd roundrect (at -1.4 0 180) (size 1.25 1.75) (layers F.Cu F.Paste F.Mask) (roundrect_rratio 0.2) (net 1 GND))
  (pad 2 smd roundrect (at 1.4 0 180) (size 1.25 1.75) (layers F.Cu F.Paste F.Mask) (roundrect_rratio 0.2) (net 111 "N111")))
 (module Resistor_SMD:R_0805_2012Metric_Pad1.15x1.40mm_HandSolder (layer F.Cu) (at 31.75 95.25)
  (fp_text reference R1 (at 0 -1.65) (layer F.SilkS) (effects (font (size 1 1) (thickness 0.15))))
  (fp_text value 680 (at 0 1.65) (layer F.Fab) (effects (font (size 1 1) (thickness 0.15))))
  (pad 1 smd roundrect (at -1.025 0) (size 1.15 1.4) (layers F.Cu F.Paste F.Mask) (roundrect_rratio 0.217391) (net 110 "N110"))
  (pad 2 smd roundrect (at 1.025 0) (size 1.15 1.4) (layers F.Cu F.Paste F.Mask) (roundrect_rratio 0.217391) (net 57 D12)))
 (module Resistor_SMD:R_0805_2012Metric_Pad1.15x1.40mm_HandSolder (layer F.Cu) (at 31.75 62.23)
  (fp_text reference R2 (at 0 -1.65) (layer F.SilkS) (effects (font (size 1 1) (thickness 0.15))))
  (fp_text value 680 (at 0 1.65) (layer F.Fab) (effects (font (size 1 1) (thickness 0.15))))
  (pad 2 smd roundrect (at 1.025 0) (size 1.15 1.4) (layers F.Cu F.Paste F.Mask) (roundrect_rratio 0.217391) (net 56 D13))
  (pad 1 smd roundrect (at -1.025 0) (size 1.15 1.4) (layers F.Cu F.Paste F.Mask) (roundrect_rratio 0.217391) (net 111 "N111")))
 (gr_circle (center 92.71 68.58) (end 94.2975 68.58) (layer Edge.Cuts) (width 0.05))
 (gr_circle (center 92.71 96.52) (end 94.2975 96.52) (layer Edge.Cuts) (width 0.05))
 (gr_circle (center 41.91 53.34) (end 43.4975 53.34) (layer Edge.Cuts) (width 0.05))
 (gr_circle (center 116.84 53.34) (end 118.4275 53.34) (layer Edge.Cuts) (width 0.05))
 (gr_circle (center 123.19 101.6) (end 124.7775 101.6) (layer Edge.Cuts) (width 0.05))
 (gr_circle (center 39.37 101.6) (end 40.9575 101.6) (layer Edge.Cuts) (width 0.05))
 (gr_line (start 128.27 50.8) (end 26.67 50.8) (layer Edge.Cuts) (width 0.05))
 (gr_line (start 128.27 104.14) (end 128.27 50.8) (layer Edge.Cuts) (width 0.05))
 (gr_line (start 127 104.14) (end 128.27 104.14) (layer Edge.Cuts) (width 0.05))
 (gr_line (start 26.67 104.14) (end 127 104.14) (layer Edge.Cuts) (width 0.05))
 (gr_line (start 26.67 50.8) (end 26.67 104.14) (layer Edge.Cuts) (width 0.05))
 (segment (start 112.395 76.2845) (end 114.3 78.1895) (width 0.508) (layer F.Cu) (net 1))
 (segment (start 112.395 74.675) (end 112.395 76.2845) (width 0.508) (layer F.Cu) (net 1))
 (segment (start 114.3 78.1895) (end 114.3 78.74) (width 0.508) (layer F.Cu) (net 1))
 (segment (start 112.6975 88.9) (end 115.57 88.9) (width 0.508) (layer F.Cu) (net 1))
 (via (at 114.3 78.74) (size 0.8) (drill 0.4) (layers F.Cu B.Cu) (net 1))
 (segment (start 115.57 88.9) (end 115.57 80.01) (width 0.508) (layer F.Cu) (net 1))
 (segment (start 115.57 80.01) (end 114.3 78.74) (width 0.508) (layer F.Cu) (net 1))
 (segment (start 114.3 78.74) (end 116.84 78.74) (width 0.508) (layer B.Cu) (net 1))
 (segment (start 116.84 92.71) (end 120.65 96.52) (width 0.508) (layer B.Cu) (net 1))
 (segment (start 116.84 78.74) (end 116.84 92.71) (width 0.508) (layer B.Cu) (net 1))
 (segment (start 49.276 57.15) (end 53.086 53.34) (width 0.254) (layer F.Cu) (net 1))
 (segment (start 33.15 57.15) (end 49.276 57.15) (width 0.254) (layer F.Cu) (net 1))
 (segment (start 65.370541 99.660541) (end 66.460001 100.750001) (width 0.254) (layer F.Cu) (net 1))
 (segment (start 34.444459 99.660541) (end 65.370541 99.660541) (width 0.254) (layer F.Cu) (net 1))
 (segment (start 33.775 100.33) (end 34.444459 99.660541) (width 0.254) (layer F.Cu) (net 1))
 (segment (start 66.460001 100.750001) (end 67.31 101.6) (width 0.254) (layer F.Cu) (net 1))
 (segment (start 33.15 100.33) (end 33.775 100.33) (width 0.254) (layer F.Cu) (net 1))
 (segment (start 70.699999 100.750001) (end 69.85 101.6) (width 0.508) (layer B.Cu) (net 1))
 (segment (start 70.704001 100.745999) (end 70.699999 100.750001) (width 0.508) (layer B.Cu) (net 1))
 (segment (start 70.704001 75.784001) (end 70.704001 100.745999) (width 0.508) (layer B.Cu) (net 1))
 (segment (start 67.31 72.39) (end 70.704001 75.784001) (width 0.508) (layer B.Cu) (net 1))
 (segment (start 53.086 54.542081) (end 53.086 53.34) (width 0.508) (layer B.Cu) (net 1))
 (segment (start 53.086 78.724) (end 53.086 54.542081) (width 0.508) (layer B.Cu) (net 1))
 (segment (start 56.912 82.55) (end 53.086 78.724) (width 0.508) (layer B.Cu) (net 1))
 (segment (start 58.42 82.55) (end 56.912 82.55) (width 0.508) (layer B.Cu) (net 1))
 (segment (start 88.655 82.922) (end 92.837 78.74) (width 0.508) (layer F.Cu) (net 1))
 (segment (start 88.655 86.36) (end 88.655 82.922) (width 0.508) (layer F.Cu) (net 1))
 (segment (start 99.06 84.963) (end 92.837 78.74) (width 0.508) (layer F.Cu) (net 1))
 (segment (start 99.06 87.63) (end 99.06 84.963) (width 0.508) (layer F.Cu) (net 1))
 (via (at 62.23 101.6) (size 0.8) (drill 0.4) (layers F.Cu B.Cu) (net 3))
 (segment (start 59.928 85.09) (end 58.42 85.09) (width 0.508) (layer B.Cu) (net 3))
 (segment (start 62.23 87.392) (end 59.928 85.09) (width 0.508) (layer B.Cu) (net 3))
 (segment (start 62.23 101.6) (end 62.23 87.392) (width 0.508) (layer B.Cu) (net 3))
 (segment (start 62.23 74.93) (end 67.31 69.85) (width 0.508) (layer B.Cu) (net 3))
 (segment (start 62.23 87.392) (end 62.23 74.93) (width 0.508) (layer B.Cu) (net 3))
 (segment (start 62.23 87.392) (end 63.208001 86.413999) (width 0.508) (layer B.Cu) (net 3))
 (segment (start 63.262 86.36) (end 63.208001 86.413999) (width 0.508) (layer B.Cu) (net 3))
 (segment (start 85.09 87.63) (end 93.98 87.63) (width 0.508) (layer F.Cu) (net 3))
 (segment (start 83.82 86.36) (end 85.09 87.63) (width 0.508) (layer F.Cu) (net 3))
 (segment (start 83.82 86.36) (end 86.605 86.36) (width 0.508) (layer F.Cu) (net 3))
 (segment (start 62.23 87.392) (end 63.262 86.36) (width 0.508) (layer B.Cu) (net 3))
 (via (at 64.77 86.36) (size 0.8) (drill 0.4) (layers F.Cu B.Cu) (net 3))
 (segment (start 63.262 86.36) (end 64.77 86.36) (width 0.508) (layer B.Cu) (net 3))
 (segment (start 82.55 86.36) (end 83.82 86.36) (width 0.508) (layer F.Cu) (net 3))
 (segment (start 64.77 86.36) (end 82.55 86.36) (width 0.508) (layer F.Cu) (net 3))
 (segment (start 109.855 80.9775) (end 110.49 81.6125) (width 0.254) (layer F.Cu) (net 62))
 (segment (start 109.855 74.675) (end 109.855 80.9775) (width 0.254) (layer F.Cu) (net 62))
 (via (at 110.49 57.15) (size 0.8) (drill 0.4) (layers F.Cu B.Cu) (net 6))
 (segment (start 96.178278 57.15) (end 110.49 57.15) (width 0.254) (layer F.Cu) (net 6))
 (segment (start 67.31 77.47) (end 75.858278 77.47) (width 0.254) (layer F.Cu) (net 6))
 (segment (start 75.858278 77.47) (end 96.178278 57.15) (width 0.254) (layer F.Cu) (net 6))
 (segment (start 110.49 57.15) (end 110.49 53.34) (width 0.254) (layer B.Cu) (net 6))
 (segment (start 111.852999 54.517001) (end 112.180001 54.189999) (width 0.254) (layer F.Cu) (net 5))
 (segment (start 93.896561 54.517001) (end 111.852999 54.517001) (width 0.254) (layer F.Cu) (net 5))
 (segment (start 73.229562 75.184) (end 93.896561 54.517001) (width 0.254) (layer F.Cu) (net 5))
 (segment (start 112.180001 54.189999) (end 113.03 53.34) (width 0.254) (layer F.Cu) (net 5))
 (segment (start 67.31 75.184) (end 73.229562 75.184) (width 0.254) (layer F.Cu) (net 5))
 (segment (start 92.837 73.66) (end 96.647 69.85) (width 0.508) (layer F.Cu) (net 17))
 (segment (start 113.665 73.0655) (end 113.665 74.675) (width 0.508) (layer F.Cu) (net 17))
 (segment (start 110.4495 69.85) (end 113.665 73.0655) (width 0.508) (layer F.Cu) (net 17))
 (segment (start 96.647 69.85) (end 110.4495 69.85) (width 0.508) (layer F.Cu) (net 17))
 (segment (start 110.49 88.5675) (end 110.8225 88.9) (width 0.254) (layer F.Cu) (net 41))
 (segment (start 110.49 86.36) (end 109.22 86.36) (width 0.254) (layer F.Cu) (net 41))
 (segment (start 110.49 86.36) (end 110.49 88.5675) (width 0.254) (layer F.Cu) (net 41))
 (segment (start 110.49 83.4875) (end 110.49 86.36) (width 0.254) (layer F.Cu) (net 41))
 (segment (start 102.87 92.71) (end 102.87 101.6) (width 0.254) (layer F.Cu) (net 41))
 (segment (start 109.22 86.36) (end 102.87 92.71) (width 0.254) (layer F.Cu) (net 41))
 (segment (start 96.52 87.63) (end 96.52 92.71) (width 0.254) (layer F.Cu) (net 2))
 (segment (start 100.33 96.52) (end 100.33 101.6) (width 0.254) (layer F.Cu) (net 2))
 (segment (start 96.52 92.71) (end 100.33 96.52) (width 0.254) (layer F.Cu) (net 2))
 (segment (start 63.246 54.542081) (end 63.246 53.34) (width 0.254) (layer F.Cu) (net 59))
 (segment (start 63.246 68.818) (end 63.246 54.542081) (width 0.254) (layer F.Cu) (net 59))
 (segment (start 59.674 72.39) (end 63.246 68.818) (width 0.254) (layer F.Cu) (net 59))
 (segment (start 58.42 72.39) (end 59.674 72.39) (width 0.254) (layer F.Cu) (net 59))
 (segment (start 32.775 94.55) (end 32.775 95.25) (width 0.254) (layer F.Cu) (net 57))
 (segment (start 32.775 79.933081) (end 32.775 94.55) (width 0.254) (layer F.Cu) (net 57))
 (segment (start 58.166 54.542081) (end 32.775 79.933081) (width 0.254) (layer F.Cu) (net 57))
 (segment (start 58.166 53.34) (end 58.166 54.542081) (width 0.254) (layer F.Cu) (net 57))
 (segment (start 33.35 62.23) (end 32.775 62.23) (width 0.254) (layer F.Cu) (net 56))
 (segment (start 47.938081 62.23) (end 33.35 62.23) (width 0.254) (layer F.Cu) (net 56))
 (segment (start 55.626 54.542081) (end 47.938081 62.23) (width 0.254) (layer F.Cu) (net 56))
 (segment (start 55.626 53.34) (end 55.626 54.542081) (width 0.254) (layer F.Cu) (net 56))
 (segment (start 30.725 99.955) (end 30.35 100.33) (width 0.254) (layer F.Cu) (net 110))
 (segment (start 30.725 95.25) (end 30.725 99.955) (width 0.254) (layer F.Cu) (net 110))
 (segment (start 30.725 57.525) (end 30.35 57.15) (width 0.254) (layer F.Cu) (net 111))
 (segment (start 30.725 62.23) (end 30.725 57.525) (width 0.254) (layer F.Cu) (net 111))
 (via (at 76.2 68.58) (size 0.8) (drill 0.4) (layers F.Cu B.Cu) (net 19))
 (segment (start 66.024 68.58) (end 76.2 68.58) (width 0.254) (layer F.Cu) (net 19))
 (segment (start 58.42 74.93) (end 59.674 74.93) (width 0.254) (layer F.Cu) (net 19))
 (segment (start 59.674 74.93) (end 66.024 68.58) (width 0.254) (layer F.Cu) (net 19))
 (segment (start 91.659999 75.022999) (end 91.987001 75.350001) (width 0.254) (layer B.Cu) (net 19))
 (segment (start 91.987001 75.350001) (end 92.837 76.2) (width 0.254) (layer B.Cu) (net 19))
 (segment (start 82.928398 68.58) (end 89.371397 75.022999) (width 0.254) (layer B.Cu) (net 19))
 (segment (start 89.371397 75.022999) (end 91.659999 75.022999) (width 0.254) (layer B.Cu) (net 19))
 (segment (start 76.2 68.58) (end 82.928398 68.58) (width 0.254) (layer B.Cu) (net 19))
 (segment (start 89.193 73.66) (end 90.297 73.66) (width 0.254) (layer F.Cu) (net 16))
 (segment (start 58.655001 78.559001) (end 84.293999 78.559001) (width 0.254) (layer F.Cu) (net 16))
 (segment (start 84.293999 78.559001) (end 89.193 73.66) (width 0.254) (layer F.Cu) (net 16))
 (segment (start 58.42 78.324) (end 58.655001 78.559001) (width 0.254) (layer F.Cu) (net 16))
 (segment (start 58.42 77.47) (end 58.42 78.324) (width 0.254) (layer F.Cu) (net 16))
 (segment (start 89.447001 77.049999) (end 90.297 76.2) (width 0.254) (layer F.Cu) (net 18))
 (segment (start 60.763001 81.099001) (end 85.397999 81.099001) (width 0.254) (layer F.Cu) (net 18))
 (segment (start 85.397999 81.099001) (end 89.447001 77.049999) (width 0.254) (layer F.Cu) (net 18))
 (segment (start 59.674 80.01) (end 60.763001 81.099001) (width 0.254) (layer F.Cu) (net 18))
 (segment (start 58.42 80.01) (end 59.674 80.01) (width 0.254) (layer F.Cu) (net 18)))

